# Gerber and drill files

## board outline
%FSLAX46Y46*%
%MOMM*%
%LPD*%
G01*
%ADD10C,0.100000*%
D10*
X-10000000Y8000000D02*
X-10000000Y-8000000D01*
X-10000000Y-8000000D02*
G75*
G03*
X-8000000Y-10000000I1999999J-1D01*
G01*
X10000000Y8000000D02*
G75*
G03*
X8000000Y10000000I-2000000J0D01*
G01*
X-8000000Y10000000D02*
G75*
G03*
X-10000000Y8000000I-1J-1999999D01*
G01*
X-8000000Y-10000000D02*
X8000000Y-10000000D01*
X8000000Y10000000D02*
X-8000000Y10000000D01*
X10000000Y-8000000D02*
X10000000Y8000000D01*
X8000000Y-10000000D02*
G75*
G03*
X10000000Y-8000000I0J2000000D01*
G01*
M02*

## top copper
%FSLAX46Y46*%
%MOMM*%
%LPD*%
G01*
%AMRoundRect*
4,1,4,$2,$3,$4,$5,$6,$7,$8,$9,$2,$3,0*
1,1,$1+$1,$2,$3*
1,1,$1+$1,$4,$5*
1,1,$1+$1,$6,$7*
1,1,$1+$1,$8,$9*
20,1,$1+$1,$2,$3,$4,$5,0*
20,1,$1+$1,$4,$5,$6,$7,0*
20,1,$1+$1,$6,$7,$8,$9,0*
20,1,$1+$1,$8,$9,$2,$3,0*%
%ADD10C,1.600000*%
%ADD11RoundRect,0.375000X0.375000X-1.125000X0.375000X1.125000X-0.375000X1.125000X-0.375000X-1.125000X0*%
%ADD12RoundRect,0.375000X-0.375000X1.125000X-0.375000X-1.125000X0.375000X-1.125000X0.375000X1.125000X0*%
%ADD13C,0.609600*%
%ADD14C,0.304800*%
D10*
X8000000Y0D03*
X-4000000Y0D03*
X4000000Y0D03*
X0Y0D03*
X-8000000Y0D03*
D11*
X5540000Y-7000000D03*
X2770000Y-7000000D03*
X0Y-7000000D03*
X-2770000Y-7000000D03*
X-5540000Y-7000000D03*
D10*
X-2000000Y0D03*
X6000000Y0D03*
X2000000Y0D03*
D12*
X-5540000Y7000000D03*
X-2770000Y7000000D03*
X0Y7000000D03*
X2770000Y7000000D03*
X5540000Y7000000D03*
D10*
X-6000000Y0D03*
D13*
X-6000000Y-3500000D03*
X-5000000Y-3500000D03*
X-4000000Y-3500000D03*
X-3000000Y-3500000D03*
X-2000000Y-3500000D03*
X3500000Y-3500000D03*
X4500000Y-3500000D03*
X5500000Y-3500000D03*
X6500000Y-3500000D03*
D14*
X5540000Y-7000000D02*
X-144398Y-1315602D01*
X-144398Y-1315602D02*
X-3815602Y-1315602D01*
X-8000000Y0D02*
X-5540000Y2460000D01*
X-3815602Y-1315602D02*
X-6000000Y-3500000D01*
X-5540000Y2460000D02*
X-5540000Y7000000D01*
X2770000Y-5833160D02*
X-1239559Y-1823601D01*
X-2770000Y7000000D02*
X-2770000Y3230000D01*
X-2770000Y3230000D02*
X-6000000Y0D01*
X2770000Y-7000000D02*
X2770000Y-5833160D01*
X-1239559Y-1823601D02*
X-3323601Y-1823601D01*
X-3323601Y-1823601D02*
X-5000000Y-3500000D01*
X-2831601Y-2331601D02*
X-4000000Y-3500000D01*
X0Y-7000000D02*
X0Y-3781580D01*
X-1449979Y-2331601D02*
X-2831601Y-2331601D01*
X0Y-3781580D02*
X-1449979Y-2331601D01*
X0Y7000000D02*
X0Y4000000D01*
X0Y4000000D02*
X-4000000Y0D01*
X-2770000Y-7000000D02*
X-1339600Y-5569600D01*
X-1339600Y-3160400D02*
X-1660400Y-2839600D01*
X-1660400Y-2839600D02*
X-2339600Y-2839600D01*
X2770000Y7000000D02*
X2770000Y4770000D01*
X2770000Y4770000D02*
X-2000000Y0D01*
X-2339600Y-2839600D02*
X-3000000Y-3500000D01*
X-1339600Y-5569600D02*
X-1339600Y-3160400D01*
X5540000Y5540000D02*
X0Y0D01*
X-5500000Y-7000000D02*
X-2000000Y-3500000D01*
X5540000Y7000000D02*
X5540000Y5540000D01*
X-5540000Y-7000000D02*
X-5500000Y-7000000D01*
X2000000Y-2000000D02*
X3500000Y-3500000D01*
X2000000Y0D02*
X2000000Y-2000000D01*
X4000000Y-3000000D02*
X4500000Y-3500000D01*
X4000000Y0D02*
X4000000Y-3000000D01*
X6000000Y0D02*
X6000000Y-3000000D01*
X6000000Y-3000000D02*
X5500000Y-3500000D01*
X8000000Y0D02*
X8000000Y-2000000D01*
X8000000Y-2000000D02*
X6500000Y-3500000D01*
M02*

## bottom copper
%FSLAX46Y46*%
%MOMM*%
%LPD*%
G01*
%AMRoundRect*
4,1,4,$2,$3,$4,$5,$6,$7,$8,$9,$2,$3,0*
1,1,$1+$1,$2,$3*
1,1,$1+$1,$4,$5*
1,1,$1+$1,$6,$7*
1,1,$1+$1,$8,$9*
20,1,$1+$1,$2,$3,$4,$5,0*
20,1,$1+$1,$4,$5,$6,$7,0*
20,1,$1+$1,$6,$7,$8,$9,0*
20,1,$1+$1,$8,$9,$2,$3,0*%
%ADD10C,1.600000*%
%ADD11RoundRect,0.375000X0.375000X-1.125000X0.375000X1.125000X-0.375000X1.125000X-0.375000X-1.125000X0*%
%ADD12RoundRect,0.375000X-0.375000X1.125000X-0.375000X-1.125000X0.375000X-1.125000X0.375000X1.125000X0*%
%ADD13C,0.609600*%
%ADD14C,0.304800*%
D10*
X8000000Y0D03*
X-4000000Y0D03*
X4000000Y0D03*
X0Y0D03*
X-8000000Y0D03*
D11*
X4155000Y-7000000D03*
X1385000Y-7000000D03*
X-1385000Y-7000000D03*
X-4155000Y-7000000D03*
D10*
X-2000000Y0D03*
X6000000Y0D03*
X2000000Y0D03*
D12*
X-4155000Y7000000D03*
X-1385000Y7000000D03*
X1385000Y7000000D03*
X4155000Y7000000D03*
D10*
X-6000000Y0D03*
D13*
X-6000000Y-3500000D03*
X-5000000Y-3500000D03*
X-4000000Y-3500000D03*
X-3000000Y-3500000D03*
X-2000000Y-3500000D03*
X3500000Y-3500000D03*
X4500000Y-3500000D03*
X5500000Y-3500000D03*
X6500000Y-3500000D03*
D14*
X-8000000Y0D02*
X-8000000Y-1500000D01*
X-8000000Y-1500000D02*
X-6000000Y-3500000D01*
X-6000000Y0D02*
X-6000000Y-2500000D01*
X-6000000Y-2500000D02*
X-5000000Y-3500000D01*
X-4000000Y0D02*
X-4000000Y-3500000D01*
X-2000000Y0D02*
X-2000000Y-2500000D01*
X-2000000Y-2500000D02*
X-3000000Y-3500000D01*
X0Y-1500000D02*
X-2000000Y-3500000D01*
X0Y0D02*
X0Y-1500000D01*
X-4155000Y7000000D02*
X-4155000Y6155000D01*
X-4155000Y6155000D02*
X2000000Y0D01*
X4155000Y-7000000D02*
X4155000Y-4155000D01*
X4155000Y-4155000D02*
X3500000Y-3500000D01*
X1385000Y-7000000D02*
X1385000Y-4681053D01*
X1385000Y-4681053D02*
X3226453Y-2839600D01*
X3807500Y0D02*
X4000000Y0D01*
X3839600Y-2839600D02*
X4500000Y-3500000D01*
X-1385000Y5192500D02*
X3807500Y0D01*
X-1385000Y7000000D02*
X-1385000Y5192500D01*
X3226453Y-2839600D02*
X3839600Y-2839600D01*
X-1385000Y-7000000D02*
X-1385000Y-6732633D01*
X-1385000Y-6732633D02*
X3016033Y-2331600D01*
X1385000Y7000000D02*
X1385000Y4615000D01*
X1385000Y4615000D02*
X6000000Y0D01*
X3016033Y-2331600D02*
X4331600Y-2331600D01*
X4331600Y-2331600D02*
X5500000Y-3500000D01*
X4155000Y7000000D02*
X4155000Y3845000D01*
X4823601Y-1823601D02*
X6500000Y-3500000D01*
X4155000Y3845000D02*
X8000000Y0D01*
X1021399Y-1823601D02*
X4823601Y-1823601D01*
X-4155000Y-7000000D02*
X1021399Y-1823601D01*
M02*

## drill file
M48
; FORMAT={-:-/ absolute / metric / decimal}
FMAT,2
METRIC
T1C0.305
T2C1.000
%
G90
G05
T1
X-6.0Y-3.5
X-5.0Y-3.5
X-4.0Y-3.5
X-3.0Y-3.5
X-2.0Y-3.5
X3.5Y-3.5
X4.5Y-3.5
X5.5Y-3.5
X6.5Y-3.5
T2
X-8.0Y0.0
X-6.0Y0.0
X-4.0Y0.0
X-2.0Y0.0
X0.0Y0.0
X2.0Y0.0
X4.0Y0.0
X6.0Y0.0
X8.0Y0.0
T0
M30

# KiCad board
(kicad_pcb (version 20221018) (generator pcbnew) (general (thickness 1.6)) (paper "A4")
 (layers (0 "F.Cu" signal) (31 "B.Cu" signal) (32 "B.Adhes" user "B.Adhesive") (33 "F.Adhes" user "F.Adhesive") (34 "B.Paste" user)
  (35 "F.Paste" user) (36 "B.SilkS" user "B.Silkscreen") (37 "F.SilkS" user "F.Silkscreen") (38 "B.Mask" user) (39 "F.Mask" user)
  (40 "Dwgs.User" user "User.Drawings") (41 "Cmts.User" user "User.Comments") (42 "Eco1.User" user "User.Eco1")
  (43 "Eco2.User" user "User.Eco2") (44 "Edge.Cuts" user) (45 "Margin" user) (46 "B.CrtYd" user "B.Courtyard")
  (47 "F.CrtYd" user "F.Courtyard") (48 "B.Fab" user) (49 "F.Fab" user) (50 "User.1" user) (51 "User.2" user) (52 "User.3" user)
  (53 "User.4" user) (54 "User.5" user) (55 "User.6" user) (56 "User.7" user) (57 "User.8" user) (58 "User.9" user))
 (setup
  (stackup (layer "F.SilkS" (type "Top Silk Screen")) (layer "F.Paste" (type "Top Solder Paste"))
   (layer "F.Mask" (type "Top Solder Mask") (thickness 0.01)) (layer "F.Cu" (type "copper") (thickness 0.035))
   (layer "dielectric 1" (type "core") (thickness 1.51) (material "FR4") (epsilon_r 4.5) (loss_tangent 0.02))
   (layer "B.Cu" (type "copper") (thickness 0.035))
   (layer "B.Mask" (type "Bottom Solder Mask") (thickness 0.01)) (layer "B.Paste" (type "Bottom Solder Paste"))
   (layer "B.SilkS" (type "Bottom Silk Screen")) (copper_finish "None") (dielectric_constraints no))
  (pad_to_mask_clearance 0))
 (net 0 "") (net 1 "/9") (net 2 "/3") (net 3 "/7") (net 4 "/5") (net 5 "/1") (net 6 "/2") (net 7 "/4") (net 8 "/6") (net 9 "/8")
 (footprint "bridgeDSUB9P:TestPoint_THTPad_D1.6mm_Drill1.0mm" (layer "F.Cu") (at 8 0)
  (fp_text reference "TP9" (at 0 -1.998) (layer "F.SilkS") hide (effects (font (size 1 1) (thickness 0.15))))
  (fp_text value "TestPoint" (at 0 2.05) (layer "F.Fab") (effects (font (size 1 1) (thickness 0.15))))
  (pad "1" thru_hole circle (at 0 0) (size 1.6 1.6) (drill 1) (layers "*.Cu" "*.Mask") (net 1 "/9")))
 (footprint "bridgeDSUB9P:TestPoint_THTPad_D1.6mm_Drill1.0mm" (layer "F.Cu") (at -4 0)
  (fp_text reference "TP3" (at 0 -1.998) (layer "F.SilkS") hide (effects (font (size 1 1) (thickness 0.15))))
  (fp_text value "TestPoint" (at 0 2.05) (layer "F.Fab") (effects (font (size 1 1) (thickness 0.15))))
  (pad "1" thru_hole circle (at 0 0) (size 1.6 1.6) (drill 1) (layers "*.Cu" "*.Mask") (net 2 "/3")))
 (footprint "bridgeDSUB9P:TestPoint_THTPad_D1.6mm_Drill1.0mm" (layer "F.Cu") (at 4 0)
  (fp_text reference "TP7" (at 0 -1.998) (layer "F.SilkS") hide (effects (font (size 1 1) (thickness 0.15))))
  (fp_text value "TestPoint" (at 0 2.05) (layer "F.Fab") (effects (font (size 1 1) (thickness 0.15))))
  (pad "1" thru_hole circle (at 0 0) (size 1.6 1.6) (drill 1) (layers "*.Cu" "*.Mask") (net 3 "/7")))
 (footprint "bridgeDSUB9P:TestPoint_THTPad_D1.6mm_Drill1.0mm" (layer "F.Cu") (at 0 0)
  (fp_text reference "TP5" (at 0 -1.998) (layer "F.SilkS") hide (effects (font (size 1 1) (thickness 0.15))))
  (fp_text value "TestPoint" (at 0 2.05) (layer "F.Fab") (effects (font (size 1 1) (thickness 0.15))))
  (pad "1" thru_hole circle (at 0 0) (size 1.6 1.6) (drill 1) (layers "*.Cu" "*.Mask") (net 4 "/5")))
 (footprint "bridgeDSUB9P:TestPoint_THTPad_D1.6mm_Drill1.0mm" (layer "F.Cu") (at -8 0)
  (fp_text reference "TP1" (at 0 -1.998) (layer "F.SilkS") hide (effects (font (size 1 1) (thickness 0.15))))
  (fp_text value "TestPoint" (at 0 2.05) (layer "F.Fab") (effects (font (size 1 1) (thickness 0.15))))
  (pad "1" thru_hole circle (at 0 0) (size 1.6 1.6) (drill 1) (layers "*.Cu" "*.Mask") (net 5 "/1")))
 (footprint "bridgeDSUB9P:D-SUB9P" (layer "F.Cu") (at 0 10 90)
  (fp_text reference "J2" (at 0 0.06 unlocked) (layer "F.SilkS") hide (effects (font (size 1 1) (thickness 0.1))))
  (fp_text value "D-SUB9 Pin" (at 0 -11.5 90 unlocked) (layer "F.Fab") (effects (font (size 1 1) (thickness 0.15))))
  (pad "1" smd roundrect (at 3 5.54 90) (size 3 1.5) (layers "F.Cu" "F.Paste" "F.Mask") (roundrect_rratio 0.25) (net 5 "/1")
   (thermal_bridge_angle 45))
  (pad "2" smd roundrect (at 3 2.77 90) (size 3 1.5) (layers "F.Cu" "F.Paste" "F.Mask") (roundrect_rratio 0.25) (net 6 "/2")
   (thermal_bridge_angle 45))
  (pad "3" smd roundrect (at 3 0 90) (size 3 1.5) (layers "F.Cu" "F.Paste" "F.Mask") (roundrect_rratio 0.25) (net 2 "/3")
   (thermal_bridge_angle 45))
  (pad "4" smd roundrect (at 3 -2.77 90) (size 3 1.5) (layers "F.Cu" "F.Paste" "F.Mask") (roundrect_rratio 0.25) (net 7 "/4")
   (thermal_bridge_angle 45))
  (pad "5" smd roundrect (at 3 -5.54 90) (size 3 1.5) (layers "F.Cu" "F.Paste" "F.Mask") (roundrect_rratio 0.25) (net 4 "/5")
   (thermal_bridge_angle 45))
  (pad "6" smd roundrect (at 3 4.155 90) (size 3 1.5) (layers "B.Cu" "B.Paste" "B.Mask") (roundrect_rratio 0.25) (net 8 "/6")
   (thermal_bridge_angle 45))
  (pad "7" smd roundrect (at 3 1.385 90) (size 3 1.5) (layers "B.Cu" "B.Paste" "B.Mask") (roundrect_rratio 0.25) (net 3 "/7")
   (thermal_bridge_angle 45))
  (pad "8" smd roundrect (at 3 -1.385 90) (size 3 1.5) (layers "B.Cu" "B.Paste" "B.Mask") (roundrect_rratio 0.25) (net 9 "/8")
   (thermal_bridge_angle 45))
  (pad "9" smd roundrect (at 3 -4.155 90) (size 3 1.5) (layers "B.Cu" "B.Paste" "B.Mask") (roundrect_rratio 0.25) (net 1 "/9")
   (thermal_bridge_angle 45)))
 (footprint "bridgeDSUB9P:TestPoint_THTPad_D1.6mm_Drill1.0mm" (layer "F.Cu") (at -2 0)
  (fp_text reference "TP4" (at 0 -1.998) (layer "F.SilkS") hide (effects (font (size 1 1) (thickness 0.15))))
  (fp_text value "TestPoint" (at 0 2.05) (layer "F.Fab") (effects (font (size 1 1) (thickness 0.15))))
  (pad "1" thru_hole circle (at 0 0) (size 1.6 1.6) (drill 1) (layers "*.Cu" "*.Mask") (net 7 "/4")))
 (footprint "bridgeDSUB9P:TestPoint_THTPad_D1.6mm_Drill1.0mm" (layer "F.Cu") (at 6 0)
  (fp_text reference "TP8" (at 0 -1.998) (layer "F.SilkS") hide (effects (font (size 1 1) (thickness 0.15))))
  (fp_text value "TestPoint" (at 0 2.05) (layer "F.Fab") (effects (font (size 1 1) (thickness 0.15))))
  (pad "1" thru_hole circle (at 0 0) (size 1.6 1.6) (drill 1) (layers "*.Cu" "*.Mask") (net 9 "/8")))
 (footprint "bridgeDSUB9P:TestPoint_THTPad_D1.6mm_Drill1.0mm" (layer "F.Cu") (at 2 0)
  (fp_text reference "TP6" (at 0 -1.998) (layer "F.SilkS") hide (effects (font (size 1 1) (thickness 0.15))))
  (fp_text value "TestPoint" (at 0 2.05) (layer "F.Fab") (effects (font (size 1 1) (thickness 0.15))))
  (pad "1" thru_hole circle (at 0 0) (size 1.6 1.6) (drill 1) (layers "*.Cu" "*.Mask") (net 8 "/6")))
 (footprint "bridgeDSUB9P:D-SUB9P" (layer "F.Cu") (at 0 -10 -90)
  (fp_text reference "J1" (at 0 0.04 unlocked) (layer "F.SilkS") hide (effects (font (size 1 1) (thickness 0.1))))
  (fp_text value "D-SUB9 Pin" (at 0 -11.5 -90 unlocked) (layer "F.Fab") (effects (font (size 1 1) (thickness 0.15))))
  (pad "1" smd roundrect (at 3 5.54 270) (size 3 1.5) (layers "F.Cu" "F.Paste" "F.Mask") (roundrect_rratio 0.25) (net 5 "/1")
   (thermal_bridge_angle 45))
  (pad "2" smd roundrect (at 3 2.77 270) (size 3 1.5) (layers "F.Cu" "F.Paste" "F.Mask") (roundrect_rratio 0.25) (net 6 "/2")
   (thermal_bridge_angle 45))
  (pad "3" smd roundrect (at 3 0 270) (size 3 1.5) (layers "F.Cu" "F.Paste" "F.Mask") (roundrect_rratio 0.25) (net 2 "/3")
   (thermal_bridge_angle 45))
  (pad "4" smd roundrect (at 3 -2.77 270) (size 3 1.5) (layers "F.Cu" "F.Paste" "F.Mask") (roundrect_rratio 0.25) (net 7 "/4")
   (thermal_bridge_angle 45))
  (pad "5" smd roundrect (at 3 -5.54 270) (size 3 1.5) (layers "F.Cu" "F.Paste" "F.Mask") (roundrect_rratio 0.25) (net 4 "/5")
   (thermal_bridge_angle 45))
  (pad "6" smd roundrect (at 3 4.155 270) (size 3 1.5) (layers "B.Cu" "B.Paste" "B.Mask") (roundrect_rratio 0.25) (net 8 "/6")
   (thermal_bridge_angle 45))
  (pad "7" smd roundrect (at 3 1.385 270) (size 3 1.5) (layers "B.Cu" "B.Paste" "B.Mask") (roundrect_rratio 0.25) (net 3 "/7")
   (thermal_bridge_angle 45))
  (pad "8" smd roundrect (at 3 -1.385 270) (size 3 1.5) (layers "B.Cu" "B.Paste" "B.Mask") (roundrect_rratio 0.25) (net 9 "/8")
   (thermal_bridge_angle 45))
  (pad "9" smd roundrect (at 3 -4.155 270) (size 3 1.5) (layers "B.Cu" "B.Paste" "B.Mask") (roundrect_rratio 0.25) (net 1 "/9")
   (thermal_bridge_angle 45)))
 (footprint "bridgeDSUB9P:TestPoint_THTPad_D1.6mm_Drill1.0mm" (layer "F.Cu") (at -6 0)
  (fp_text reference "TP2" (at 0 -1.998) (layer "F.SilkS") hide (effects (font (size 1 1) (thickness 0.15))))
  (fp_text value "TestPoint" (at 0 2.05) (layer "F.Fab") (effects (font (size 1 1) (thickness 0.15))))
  (pad "1" thru_hole circle (at 0 0) (size 1.6 1.6) (drill 1) (layers "*.Cu" "*.Mask") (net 6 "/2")))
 (gr_line (start -10 -8) (end -10 8) (stroke (width 0.1) (type default)) (layer "Edge.Cuts"))
 (gr_arc (start -8 10) (mid -9.414214 9.414214) (end -10 8) (stroke (width 0.1) (type default)) (layer "Edge.Cuts"))
 (gr_arc (start 8 -10) (mid 9.414214 -9.414214) (end 10 -8) (stroke (width 0.1) (type default)) (layer "Edge.Cuts"))
 (gr_arc (start -10 -8) (mid -9.414214 -9.414214) (end -8 -10) (stroke (width 0.1) (type default)) (layer "Edge.Cuts"))
 (gr_line (start -8 10) (end 8 10) (stroke (width 0.1) (type default)) (layer "Edge.Cuts"))
 (gr_line (start 8 -10) (end -8 -10) (stroke (width 0.1) (type default)) (layer "Edge.Cuts"))
 (gr_line (start 10 8) (end 10 -8) (stroke (width 0.1) (type default)) (layer "Edge.Cuts"))
 (gr_arc (start 10 8) (mid 9.414214 9.414214) (end 8 10) (stroke (width 0.1) (type default)) (layer "Edge.Cuts"))
 (segment (start 5.54 7) (end -0.144398 1.315602) (width 0.3048) (layer "F.Cu") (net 5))
 (segment (start -0.144398 1.315602) (end -3.815602 1.315602) (width 0.3048) (layer "F.Cu") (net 5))
 (segment (start -8 0) (end -5.54 -2.46) (width 0.3048) (layer "F.Cu") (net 5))
 (segment (start -3.815602 1.315602) (end -6 3.5) (width 0.3048) (layer "F.Cu") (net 5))
 (segment (start -5.54 -2.46) (end -5.54 -7) (width 0.3048) (layer "F.Cu") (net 5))
 (via (at -6 3.5) (size 0.6096) (drill 0.3048) (layers "F.Cu" "B.Cu") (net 5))
 (segment (start -8 0) (end -8 1.5) (width 0.3048) (layer "B.Cu") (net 5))
 (segment (start -8 1.5) (end -6 3.5) (width 0.3048) (layer "B.Cu") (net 5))
 (segment (start 2.77 5.83316) (end -1.239559 1.823601) (width 0.3048) (layer "F.Cu") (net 6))
 (segment (start -2.77 -7) (end -2.77 -3.23) (width 0.3048) (layer "F.Cu") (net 6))
 (segment (start -2.77 -3.23) (end -6 0) (width 0.3048) (layer "F.Cu") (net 6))
 (segment (start 2.77 7) (end 2.77 5.83316) (width 0.3048) (layer "F.Cu") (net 6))
 (segment (start -1.239559 1.823601) (end -3.323601 1.823601) (width 0.3048) (layer "F.Cu") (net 6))
 (segment (start -3.323601 1.823601) (end -5 3.5) (width 0.3048) (layer "F.Cu") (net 6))
 (via (at -5 3.5) (size 0.6096) (drill 0.3048) (layers "F.Cu" "B.Cu") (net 6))
 (segment (start -6 0) (end -6 2.5) (width 0.3048) (layer "B.Cu") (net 6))
 (segment (start -6 2.5) (end -5 3.5) (width 0.3048) (layer "B.Cu") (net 6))
 (segment (start -2.831601 2.331601) (end -4 3.5) (width 0.3048) (layer "F.Cu") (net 2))
 (segment (start 0 7) (end 0 3.78158) (width 0.3048) (layer "F.Cu") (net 2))
 (segment (start -1.449979 2.331601) (end -2.831601 2.331601) (width 0.3048) (layer "F.Cu") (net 2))
 (segment (start 0 3.78158) (end -1.449979 2.331601) (width 0.3048) (layer "F.Cu") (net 2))
 (segment (start 0 -7) (end 0 -4) (width 0.3048) (layer "F.Cu") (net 2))
 (segment (start 0 -4) (end -4 0) (width 0.3048) (layer "F.Cu") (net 2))
 (via (at -4 3.5) (size 0.6096) (drill 0.3048) (layers "F.Cu" "B.Cu") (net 2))
 (segment (start -4 0) (end -4 3.5) (width 0.3048) (layer "B.Cu") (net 2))
 (segment (start -2.77 7) (end -1.3396 5.5696) (width 0.3048) (layer "F.Cu") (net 7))
 (segment (start -1.3396 3.1604) (end -1.6604 2.8396) (width 0.3048) (layer "F.Cu") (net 7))
 (segment (start -1.6604 2.8396) (end -2.3396 2.8396) (width 0.3048) (layer "F.Cu") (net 7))
 (segment (start 2.77 -7) (end 2.77 -4.77) (width 0.3048) (layer "F.Cu") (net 7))
 (segment (start 2.77 -4.77) (end -2 0) (width 0.3048) (layer "F.Cu") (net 7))
 (segment (start -2.3396 2.8396) (end -3 3.5) (width 0.3048) (layer "F.Cu") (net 7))
 (segment (start -1.3396 5.5696) (end -1.3396 3.1604) (width 0.3048) (layer "F.Cu") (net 7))
 (via (at -3 3.5) (size 0.6096) (drill 0.3048) (layers "F.Cu" "B.Cu") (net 7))
 (segment (start -2 0) (end -2 2.5) (width 0.3048) (layer "B.Cu") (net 7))
 (segment (start -2 2.5) (end -3 3.5) (width 0.3048) (layer "B.Cu") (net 7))
 (segment (start 5.54 -5.54) (end 0 0) (width 0.3048) (layer "F.Cu") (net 4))
 (segment (start -5.5 7) (end -2 3.5) (width 0.3048) (layer "F.Cu") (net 4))
 (segment (start 5.54 -7) (end 5.54 -5.54) (width 0.3048) (layer "F.Cu") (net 4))
 (segment (start -5.54 7) (end -5.5 7) (width 0.3048) (layer "F.Cu") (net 4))
 (via (at -2 3.5) (size 0.6096) (drill 0.3048) (layers "F.Cu" "B.Cu") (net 4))
 (segment (start 0 1.5) (end -2 3.5) (width 0.3048) (layer "B.Cu") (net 4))
 (segment (start 0 0) (end 0 1.5) (width 0.3048) (layer "B.Cu") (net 4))
 (segment (start 2 2) (end 3.5 3.5) (width 0.3048) (layer "F.Cu") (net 8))
 (segment (start 2 0) (end 2 2) (width 0.3048) (layer "F.Cu") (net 8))
 (via (at 3.5 3.5) (size 0.6096) (drill 0.3048) (layers "F.Cu" "B.Cu") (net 8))
 (segment (start -4.155 -7) (end -4.155 -6.155) (width 0.3048) (layer "B.Cu") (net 8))
 (segment (start -4.155 -6.155) (end 2 0) (width 0.3048) (layer "B.Cu") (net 8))
 (segment (start 4.155 7) (end 4.155 4.155) (width 0.3048) (layer "B.Cu") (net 8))
 (segment (start 4.155 4.155) (end 3.5 3.5) (width 0.3048) (layer "B.Cu") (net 8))
 (segment (start 4 3) (end 4.5 3.5) (width 0.3048) (layer "F.Cu") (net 3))
 (segment (start 4 0) (end 4 3) (width 0.3048) (layer "F.Cu") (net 3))
 (via (at 4.5 3.5) (size 0.6096) (drill 0.3048) (layers "F.Cu" "B.Cu") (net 3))
 (segment (start 1.385 7) (end 1.385 4.681053) (width 0.3048) (layer "B.Cu") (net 3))
 (segment (start 1.385 4.681053) (end 3.226453 2.8396) (width 0.3048) (layer "B.Cu") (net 3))
 (segment (start 3.8075 0) (end 4 0) (width 0.3048) (layer "B.Cu") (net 3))
 (segment (start 3.8396 2.8396) (end 4.5 3.5) (width 0.3048) (layer "B.Cu") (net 3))
 (segment (start -1.385 -5.1925) (end 3.8075 0) (width 0.3048) (layer "B.Cu") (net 3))
 (segment (start -1.385 -7) (end -1.385 -5.1925) (width 0.3048) (layer "B.Cu") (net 3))
 (segment (start 3.226453 2.8396) (end 3.8396 2.8396) (width 0.3048) (layer "B.Cu") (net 3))
 (segment (start 6 0) (end 6 3) (width 0.3048) (layer "F.Cu") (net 9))
 (segment (start 6 3) (end 5.5 3.5) (width 0.3048) (layer "F.Cu") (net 9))
 (via (at 5.5 3.5) (size 0.6096) (drill 0.3048) (layers "F.Cu" "B.Cu") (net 9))
 (segment (start -1.385 7) (end -1.385 6.732633) (width 0.3048) (layer "B.Cu") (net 9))
 (segment (start -1.385 6.732633) (end 3.016033 2.3316) (width 0.3048) (layer "B.Cu") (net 9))
 (segment (start 1.385 -7) (end 1.385 -4.615) (width 0.3048) (layer "B.Cu") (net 9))
 (segment (start 1.385 -4.615) (end 6 0) (width 0.3048) (layer "B.Cu") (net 9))
 (segment (start 3.016033 2.3316) (end 4.3316 2.3316) (width 0.3048) (layer "B.Cu") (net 9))
 (segment (start 4.3316 2.3316) (end 5.5 3.5) (width 0.3048) (layer "B.Cu") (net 9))
 (segment (start 8 0) (end 8 2) (width 0.3048) (layer "F.Cu") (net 1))
 (segment (start 8 2) (end 6.5 3.5) (width 0.3048) (layer "F.Cu") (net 1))
 (via (at 6.5 3.5) (size 0.6096) (drill 0.3048) (layers "F.Cu" "B.Cu") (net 1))
 (segment (start 4.155 -7) (end 4.155 -3.845) (width 0.3048) (layer "B.Cu") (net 1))
 (segment (start 4.823601 1.823601) (end 6.5 3.5) (width 0.3048) (layer "B.Cu") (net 1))
 (segment (start 4.155 -3.845) (end 8 0) (width 0.3048) (layer "B.Cu") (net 1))
 (segment (start 1.021399 1.823601) (end 4.823601 1.823601) (width 0.3048) (layer "B.Cu") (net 1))
 (segment (start -4.155 7) (end 1.021399 1.823601) (width 0.3048) (layer "B.Cu") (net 1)))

